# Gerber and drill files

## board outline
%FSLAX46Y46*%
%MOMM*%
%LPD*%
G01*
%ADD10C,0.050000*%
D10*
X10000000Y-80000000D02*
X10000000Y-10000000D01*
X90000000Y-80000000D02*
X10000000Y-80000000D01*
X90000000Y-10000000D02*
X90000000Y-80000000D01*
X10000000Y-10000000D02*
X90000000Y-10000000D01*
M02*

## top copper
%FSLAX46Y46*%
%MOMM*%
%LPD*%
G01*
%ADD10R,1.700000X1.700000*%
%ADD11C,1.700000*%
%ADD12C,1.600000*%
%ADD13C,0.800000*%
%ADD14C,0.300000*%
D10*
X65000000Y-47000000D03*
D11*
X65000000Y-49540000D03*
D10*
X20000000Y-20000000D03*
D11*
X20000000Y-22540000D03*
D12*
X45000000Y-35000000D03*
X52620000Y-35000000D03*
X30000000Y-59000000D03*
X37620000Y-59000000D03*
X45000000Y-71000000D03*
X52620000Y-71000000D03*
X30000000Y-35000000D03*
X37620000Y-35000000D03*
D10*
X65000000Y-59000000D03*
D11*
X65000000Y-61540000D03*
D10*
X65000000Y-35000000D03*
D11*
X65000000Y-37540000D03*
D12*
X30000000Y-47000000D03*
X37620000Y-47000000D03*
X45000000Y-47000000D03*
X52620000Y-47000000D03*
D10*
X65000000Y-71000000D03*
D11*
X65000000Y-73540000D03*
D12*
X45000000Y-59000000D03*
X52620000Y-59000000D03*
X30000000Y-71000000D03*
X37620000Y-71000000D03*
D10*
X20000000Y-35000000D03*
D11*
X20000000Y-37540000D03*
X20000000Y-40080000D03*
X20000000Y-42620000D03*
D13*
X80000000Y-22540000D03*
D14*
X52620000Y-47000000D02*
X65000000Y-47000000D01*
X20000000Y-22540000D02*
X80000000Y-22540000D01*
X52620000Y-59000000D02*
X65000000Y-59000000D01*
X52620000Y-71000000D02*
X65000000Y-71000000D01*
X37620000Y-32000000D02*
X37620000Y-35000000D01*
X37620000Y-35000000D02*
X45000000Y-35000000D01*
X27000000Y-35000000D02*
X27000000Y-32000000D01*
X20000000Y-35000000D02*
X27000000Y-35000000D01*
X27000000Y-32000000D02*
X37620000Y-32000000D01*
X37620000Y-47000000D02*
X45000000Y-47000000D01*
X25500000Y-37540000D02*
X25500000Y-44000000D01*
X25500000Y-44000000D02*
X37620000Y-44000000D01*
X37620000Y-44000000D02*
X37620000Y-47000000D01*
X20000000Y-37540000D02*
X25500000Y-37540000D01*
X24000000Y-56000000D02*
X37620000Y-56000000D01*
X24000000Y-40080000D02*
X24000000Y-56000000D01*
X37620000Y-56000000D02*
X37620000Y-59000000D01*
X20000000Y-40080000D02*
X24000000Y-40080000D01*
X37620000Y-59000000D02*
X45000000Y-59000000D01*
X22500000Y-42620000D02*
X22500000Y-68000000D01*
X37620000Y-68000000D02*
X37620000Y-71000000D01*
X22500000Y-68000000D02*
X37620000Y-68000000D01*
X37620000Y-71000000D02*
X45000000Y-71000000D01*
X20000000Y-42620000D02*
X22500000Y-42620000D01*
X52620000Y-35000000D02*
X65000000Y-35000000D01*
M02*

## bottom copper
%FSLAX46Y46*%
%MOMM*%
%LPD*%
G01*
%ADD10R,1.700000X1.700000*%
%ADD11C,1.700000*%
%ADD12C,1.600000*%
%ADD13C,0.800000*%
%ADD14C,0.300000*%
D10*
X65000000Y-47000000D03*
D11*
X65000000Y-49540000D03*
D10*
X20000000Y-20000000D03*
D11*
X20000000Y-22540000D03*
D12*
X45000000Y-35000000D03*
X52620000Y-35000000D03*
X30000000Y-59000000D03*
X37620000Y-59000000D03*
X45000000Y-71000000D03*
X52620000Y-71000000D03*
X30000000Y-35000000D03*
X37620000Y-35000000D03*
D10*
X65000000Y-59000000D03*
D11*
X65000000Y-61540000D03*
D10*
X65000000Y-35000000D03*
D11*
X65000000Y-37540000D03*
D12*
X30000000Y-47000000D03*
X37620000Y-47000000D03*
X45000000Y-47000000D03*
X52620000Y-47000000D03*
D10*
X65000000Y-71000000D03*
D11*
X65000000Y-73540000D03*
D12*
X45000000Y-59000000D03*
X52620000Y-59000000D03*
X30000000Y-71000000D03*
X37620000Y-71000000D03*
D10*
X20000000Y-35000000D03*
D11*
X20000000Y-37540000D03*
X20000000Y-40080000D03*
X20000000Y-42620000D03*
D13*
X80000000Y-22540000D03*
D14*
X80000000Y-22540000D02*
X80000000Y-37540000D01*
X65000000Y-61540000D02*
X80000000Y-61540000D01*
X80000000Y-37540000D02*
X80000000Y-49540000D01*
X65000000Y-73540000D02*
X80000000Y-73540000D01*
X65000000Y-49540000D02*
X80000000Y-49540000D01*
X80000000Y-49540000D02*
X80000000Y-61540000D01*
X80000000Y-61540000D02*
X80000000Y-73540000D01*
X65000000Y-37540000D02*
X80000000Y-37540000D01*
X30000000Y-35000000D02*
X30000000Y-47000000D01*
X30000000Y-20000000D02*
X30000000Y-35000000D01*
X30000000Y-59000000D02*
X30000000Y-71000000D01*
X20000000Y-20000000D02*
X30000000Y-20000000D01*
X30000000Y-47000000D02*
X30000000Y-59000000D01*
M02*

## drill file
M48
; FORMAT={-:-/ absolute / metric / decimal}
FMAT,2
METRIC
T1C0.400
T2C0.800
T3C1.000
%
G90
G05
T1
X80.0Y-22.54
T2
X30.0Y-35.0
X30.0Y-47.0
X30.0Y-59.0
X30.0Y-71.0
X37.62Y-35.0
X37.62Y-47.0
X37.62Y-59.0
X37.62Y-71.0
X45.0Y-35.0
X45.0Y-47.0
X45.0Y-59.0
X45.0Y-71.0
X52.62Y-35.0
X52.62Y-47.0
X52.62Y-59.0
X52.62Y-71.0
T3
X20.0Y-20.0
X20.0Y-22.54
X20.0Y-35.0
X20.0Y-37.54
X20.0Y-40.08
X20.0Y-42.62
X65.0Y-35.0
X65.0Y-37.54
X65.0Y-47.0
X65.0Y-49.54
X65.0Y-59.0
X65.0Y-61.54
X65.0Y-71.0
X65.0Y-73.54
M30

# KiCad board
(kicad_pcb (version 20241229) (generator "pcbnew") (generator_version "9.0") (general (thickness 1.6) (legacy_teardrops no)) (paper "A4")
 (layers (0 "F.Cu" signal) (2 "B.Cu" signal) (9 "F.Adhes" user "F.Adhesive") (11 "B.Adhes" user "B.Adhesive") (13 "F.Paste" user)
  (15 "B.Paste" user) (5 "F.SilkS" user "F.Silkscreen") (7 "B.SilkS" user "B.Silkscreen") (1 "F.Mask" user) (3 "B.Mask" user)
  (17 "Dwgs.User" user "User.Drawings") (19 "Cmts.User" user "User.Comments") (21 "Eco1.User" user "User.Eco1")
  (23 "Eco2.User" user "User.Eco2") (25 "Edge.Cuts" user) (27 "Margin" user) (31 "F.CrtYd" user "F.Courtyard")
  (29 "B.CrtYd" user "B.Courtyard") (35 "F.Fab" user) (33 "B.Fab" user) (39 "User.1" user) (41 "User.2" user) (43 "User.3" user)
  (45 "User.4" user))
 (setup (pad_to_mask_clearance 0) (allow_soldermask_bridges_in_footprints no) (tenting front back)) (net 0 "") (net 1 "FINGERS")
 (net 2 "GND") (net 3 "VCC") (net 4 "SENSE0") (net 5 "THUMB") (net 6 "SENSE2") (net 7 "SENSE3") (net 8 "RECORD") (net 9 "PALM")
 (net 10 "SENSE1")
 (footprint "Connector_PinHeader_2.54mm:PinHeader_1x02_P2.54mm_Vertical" (layer "F.Cu") (at 65 47)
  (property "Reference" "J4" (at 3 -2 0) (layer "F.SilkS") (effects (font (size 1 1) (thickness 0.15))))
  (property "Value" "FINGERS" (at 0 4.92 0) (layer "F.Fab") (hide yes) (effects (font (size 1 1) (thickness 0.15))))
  (pad "1" thru_hole rect (at 0 0) (size 1.7 1.7) (drill 1) (layers "*.Cu" "*.Mask") (remove_unused_layers no) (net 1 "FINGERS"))
  (pad "2" thru_hole circle (at 0 2.54) (size 1.7 1.7) (drill 1) (layers "*.Cu" "*.Mask") (remove_unused_layers no) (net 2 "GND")))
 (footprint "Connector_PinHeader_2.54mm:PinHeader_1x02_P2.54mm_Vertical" (layer "F.Cu") (at 20 20)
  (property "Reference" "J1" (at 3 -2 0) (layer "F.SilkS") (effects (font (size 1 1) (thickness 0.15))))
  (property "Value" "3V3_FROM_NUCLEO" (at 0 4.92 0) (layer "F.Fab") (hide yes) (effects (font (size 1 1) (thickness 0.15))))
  (pad "1" thru_hole rect (at 0 0) (size 1.7 1.7) (drill 1) (layers "*.Cu" "*.Mask") (remove_unused_layers no) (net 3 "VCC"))
  (pad "2" thru_hole circle (at 0 2.54) (size 1.7 1.7) (drill 1) (layers "*.Cu" "*.Mask") (remove_unused_layers no) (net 2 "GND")))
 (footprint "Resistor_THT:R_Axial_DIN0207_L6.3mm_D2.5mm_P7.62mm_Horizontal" (layer "F.Cu") (at 45 35)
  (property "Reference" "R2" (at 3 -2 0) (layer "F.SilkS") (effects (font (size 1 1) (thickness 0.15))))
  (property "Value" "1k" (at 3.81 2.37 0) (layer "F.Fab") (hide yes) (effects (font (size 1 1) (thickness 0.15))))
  (pad "1" thru_hole circle (at 0 0) (size 1.6 1.6) (drill 0.8) (layers "*.Cu" "*.Mask") (remove_unused_layers no) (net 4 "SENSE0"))
  (pad "2" thru_hole circle (at 7.62 0) (size 1.6 1.6) (drill 0.8) (layers "*.Cu" "*.Mask") (remove_unused_layers no) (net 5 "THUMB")))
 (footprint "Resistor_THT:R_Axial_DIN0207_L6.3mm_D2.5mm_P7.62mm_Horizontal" (layer "F.Cu") (at 30 59)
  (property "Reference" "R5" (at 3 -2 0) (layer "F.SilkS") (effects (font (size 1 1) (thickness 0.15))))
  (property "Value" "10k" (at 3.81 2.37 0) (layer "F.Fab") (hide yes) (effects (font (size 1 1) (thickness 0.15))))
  (pad "1" thru_hole circle (at 0 0) (size 1.6 1.6) (drill 0.8) (layers "*.Cu" "*.Mask") (remove_unused_layers no) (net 3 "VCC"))
  (pad "2" thru_hole circle (at 7.62 0) (size 1.6 1.6) (drill 0.8) (layers "*.Cu" "*.Mask") (remove_unused_layers no) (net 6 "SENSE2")))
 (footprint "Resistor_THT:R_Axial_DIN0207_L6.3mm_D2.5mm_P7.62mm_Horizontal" (layer "F.Cu") (at 45 71)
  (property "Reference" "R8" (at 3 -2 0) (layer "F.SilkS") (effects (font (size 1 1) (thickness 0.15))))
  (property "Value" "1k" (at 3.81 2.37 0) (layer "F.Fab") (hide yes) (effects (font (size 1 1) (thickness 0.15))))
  (pad "1" thru_hole circle (at 0 0) (size 1.6 1.6) (drill 0.8) (layers "*.Cu" "*.Mask") (remove_unused_layers no) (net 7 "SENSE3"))
  (pad "2" thru_hole circle (at 7.62 0) (size 1.6 1.6) (drill 0.8) (layers "*.Cu" "*.Mask") (remove_unused_layers no) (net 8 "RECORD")))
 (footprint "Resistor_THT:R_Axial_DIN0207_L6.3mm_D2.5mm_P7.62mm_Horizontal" (layer "F.Cu") (at 30 35)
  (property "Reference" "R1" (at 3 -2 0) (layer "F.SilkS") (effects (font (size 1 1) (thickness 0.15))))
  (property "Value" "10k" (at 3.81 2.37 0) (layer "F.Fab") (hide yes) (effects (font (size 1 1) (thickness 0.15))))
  (pad "1" thru_hole circle (at 0 0) (size 1.6 1.6) (drill 0.8) (layers "*.Cu" "*.Mask") (remove_unused_layers no) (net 3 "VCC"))
  (pad "2" thru_hole circle (at 7.62 0) (size 1.6 1.6) (drill 0.8) (layers "*.Cu" "*.Mask") (remove_unused_layers no) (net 4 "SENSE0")))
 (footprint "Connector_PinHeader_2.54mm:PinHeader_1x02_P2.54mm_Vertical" (layer "F.Cu") (at 65 59)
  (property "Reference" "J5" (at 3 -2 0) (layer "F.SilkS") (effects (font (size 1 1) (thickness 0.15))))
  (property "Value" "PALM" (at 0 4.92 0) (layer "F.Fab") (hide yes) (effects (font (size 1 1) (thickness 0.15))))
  (pad "1" thru_hole rect (at 0 0) (size 1.7 1.7) (drill 1) (layers "*.Cu" "*.Mask") (remove_unused_layers no) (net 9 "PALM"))
  (pad "2" thru_hole circle (at 0 2.54) (size 1.7 1.7) (drill 1) (layers "*.Cu" "*.Mask") (remove_unused_layers no) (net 2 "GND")))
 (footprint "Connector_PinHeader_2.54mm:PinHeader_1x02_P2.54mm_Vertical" (layer "F.Cu") (at 65 35)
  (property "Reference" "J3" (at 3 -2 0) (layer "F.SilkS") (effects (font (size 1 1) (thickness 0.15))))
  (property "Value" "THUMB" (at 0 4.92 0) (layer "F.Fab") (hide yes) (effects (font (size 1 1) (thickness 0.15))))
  (pad "1" thru_hole rect (at 0 0) (size 1.7 1.7) (drill 1) (layers "*.Cu" "*.Mask") (remove_unused_layers no) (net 5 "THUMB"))
  (pad "2" thru_hole circle (at 0 2.54) (size 1.7 1.7) (drill 1) (layers "*.Cu" "*.Mask") (remove_unused_layers no) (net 2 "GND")))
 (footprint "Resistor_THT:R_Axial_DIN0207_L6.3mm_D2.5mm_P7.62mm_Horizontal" (layer "F.Cu") (at 30 47)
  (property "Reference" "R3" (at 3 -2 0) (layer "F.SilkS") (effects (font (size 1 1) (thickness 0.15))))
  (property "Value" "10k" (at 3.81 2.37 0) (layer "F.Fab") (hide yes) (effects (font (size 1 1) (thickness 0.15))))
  (pad "1" thru_hole circle (at 0 0) (size 1.6 1.6) (drill 0.8) (layers "*.Cu" "*.Mask") (remove_unused_layers no) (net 3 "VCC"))
  (pad "2" thru_hole circle (at 7.62 0) (size 1.6 1.6) (drill 0.8) (layers "*.Cu" "*.Mask") (remove_unused_layers no) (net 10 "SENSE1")))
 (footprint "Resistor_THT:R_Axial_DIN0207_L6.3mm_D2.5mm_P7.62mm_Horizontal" (layer "F.Cu") (at 45 47)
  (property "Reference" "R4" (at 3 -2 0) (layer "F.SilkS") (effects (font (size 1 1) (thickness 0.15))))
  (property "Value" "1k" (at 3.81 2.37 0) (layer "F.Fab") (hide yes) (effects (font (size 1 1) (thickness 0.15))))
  (pad "1" thru_hole circle (at 0 0) (size 1.6 1.6) (drill 0.8) (layers "*.Cu" "*.Mask") (remove_unused_layers no) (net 10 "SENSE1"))
  (pad "2" thru_hole circle (at 7.62 0) (size 1.6 1.6) (drill 0.8) (layers "*.Cu" "*.Mask") (remove_unused_layers no) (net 1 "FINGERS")))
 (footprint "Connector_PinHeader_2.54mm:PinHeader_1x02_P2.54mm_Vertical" (layer "F.Cu") (at 65 71)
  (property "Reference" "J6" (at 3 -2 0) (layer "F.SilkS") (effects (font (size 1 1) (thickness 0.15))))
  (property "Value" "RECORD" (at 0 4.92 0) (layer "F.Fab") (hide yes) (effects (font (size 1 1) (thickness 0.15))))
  (pad "1" thru_hole rect (at 0 0) (size 1.7 1.7) (drill 1) (layers "*.Cu" "*.Mask") (remove_unused_layers no) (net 8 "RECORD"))
  (pad "2" thru_hole circle (at 0 2.54) (size 1.7 1.7) (drill 1) (layers "*.Cu" "*.Mask") (remove_unused_layers no) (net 2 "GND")))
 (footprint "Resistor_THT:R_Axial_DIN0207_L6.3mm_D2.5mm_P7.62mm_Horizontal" (layer "F.Cu") (at 45 59)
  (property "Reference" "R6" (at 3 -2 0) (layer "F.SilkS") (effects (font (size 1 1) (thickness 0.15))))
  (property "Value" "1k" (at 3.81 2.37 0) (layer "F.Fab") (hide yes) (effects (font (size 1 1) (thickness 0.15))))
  (pad "1" thru_hole circle (at 0 0) (size 1.6 1.6) (drill 0.8) (layers "*.Cu" "*.Mask") (remove_unused_layers no) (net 6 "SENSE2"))
  (pad "2" thru_hole circle (at 7.62 0) (size 1.6 1.6) (drill 0.8) (layers "*.Cu" "*.Mask") (remove_unused_layers no) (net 9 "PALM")))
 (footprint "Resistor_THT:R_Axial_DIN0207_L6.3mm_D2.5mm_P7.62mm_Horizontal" (layer "F.Cu") (at 30 71)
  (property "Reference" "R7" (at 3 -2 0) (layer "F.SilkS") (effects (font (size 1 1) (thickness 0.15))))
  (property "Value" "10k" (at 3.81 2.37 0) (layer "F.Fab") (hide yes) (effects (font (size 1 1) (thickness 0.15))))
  (pad "1" thru_hole circle (at 0 0) (size 1.6 1.6) (drill 0.8) (layers "*.Cu" "*.Mask") (remove_unused_layers no) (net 3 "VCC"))
  (pad "2" thru_hole circle (at 7.62 0) (size 1.6 1.6) (drill 0.8) (layers "*.Cu" "*.Mask") (remove_unused_layers no) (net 7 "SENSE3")))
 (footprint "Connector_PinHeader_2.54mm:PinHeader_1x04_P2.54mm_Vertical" (layer "F.Cu") (at 20 35)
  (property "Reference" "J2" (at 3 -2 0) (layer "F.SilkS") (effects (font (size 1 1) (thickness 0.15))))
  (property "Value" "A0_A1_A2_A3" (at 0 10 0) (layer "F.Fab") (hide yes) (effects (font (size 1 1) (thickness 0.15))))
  (pad "1" thru_hole rect (at 0 0) (size 1.7 1.7) (drill 1) (layers "*.Cu" "*.Mask") (remove_unused_layers no) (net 4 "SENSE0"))
  (pad "2" thru_hole circle (at 0 2.54) (size 1.7 1.7) (drill 1) (layers "*.Cu" "*.Mask") (remove_unused_layers no) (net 10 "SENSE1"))
  (pad "3" thru_hole circle (at 0 5.08) (size 1.7 1.7) (drill 1) (layers "*.Cu" "*.Mask") (remove_unused_layers no) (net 6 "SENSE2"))
  (pad "4" thru_hole circle (at 0 7.62) (size 1.7 1.7) (drill 1) (layers "*.Cu" "*.Mask") (remove_unused_layers no) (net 7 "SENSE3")))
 (gr_line (start 10 80) (end 10 10) (stroke (width 0.05) (type default)) (layer "Edge.Cuts"))
 (gr_line (start 90 80) (end 10 80) (stroke (width 0.05) (type default)) (layer "Edge.Cuts"))
 (gr_line (start 90 10) (end 90 80) (stroke (width 0.05) (type default)) (layer "Edge.Cuts"))
 (gr_line (start 10 10) (end 90 10) (stroke (width 0.05) (type default)) (layer "Edge.Cuts"))
 (segment (start 52.62 47) (end 65 47) (width 0.3) (layer "F.Cu") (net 1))
 (segment (start 20 22.54) (end 80 22.54) (width 0.3) (layer "F.Cu") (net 2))
 (via (at 80 22.54) (size 0.8) (drill 0.4) (layers "F.Cu" "B.Cu") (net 2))
 (segment (start 80 22.54) (end 80 37.54) (width 0.3) (layer "B.Cu") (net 2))
 (segment (start 65 61.54) (end 80 61.54) (width 0.3) (layer "B.Cu") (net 2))
 (segment (start 80 37.54) (end 80 49.54) (width 0.3) (layer "B.Cu") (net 2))
 (segment (start 65 73.54) (end 80 73.54) (width 0.3) (layer "B.Cu") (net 2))
 (segment (start 65 49.54) (end 80 49.54) (width 0.3) (layer "B.Cu") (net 2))
 (segment (start 80 49.54) (end 80 61.54) (width 0.3) (layer "B.Cu") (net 2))
 (segment (start 80 61.54) (end 80 73.54) (width 0.3) (layer "B.Cu") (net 2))
 (segment (start 65 37.54) (end 80 37.54) (width 0.3) (layer "B.Cu") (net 2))
 (segment (start 52.62 59) (end 65 59) (width 0.3) (layer "F.Cu") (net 9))
 (segment (start 52.62 71) (end 65 71) (width 0.3) (layer "F.Cu") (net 8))
 (segment (start 37.62 32) (end 37.62 35) (width 0.3) (layer "F.Cu") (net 4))
 (segment (start 37.62 35) (end 45 35) (width 0.3) (layer "F.Cu") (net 4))
 (segment (start 27 35) (end 27 32) (width 0.3) (layer "F.Cu") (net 4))
 (segment (start 20 35) (end 27 35) (width 0.3) (layer "F.Cu") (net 4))
 (segment (start 27 32) (end 37.62 32) (width 0.3) (layer "F.Cu") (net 4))
 (segment (start 37.62 47) (end 45 47) (width 0.3) (layer "F.Cu") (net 10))
 (segment (start 25.5 37.54) (end 25.5 44) (width 0.3) (layer "F.Cu") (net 10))
 (segment (start 25.5 44) (end 37.62 44) (width 0.3) (layer "F.Cu") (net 10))
 (segment (start 37.62 44) (end 37.62 47) (width 0.3) (layer "F.Cu") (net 10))
 (segment (start 20 37.54) (end 25.5 37.54) (width 0.3) (layer "F.Cu") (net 10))
 (segment (start 24 56) (end 37.62 56) (width 0.3) (layer "F.Cu") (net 6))
 (segment (start 24 40.08) (end 24 56) (width 0.3) (layer "F.Cu") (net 6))
 (segment (start 37.62 56) (end 37.62 59) (width 0.3) (layer "F.Cu") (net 6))
 (segment (start 20 40.08) (end 24 40.08) (width 0.3) (layer "F.Cu") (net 6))
 (segment (start 37.62 59) (end 45 59) (width 0.3) (layer "F.Cu") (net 6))
 (segment (start 22.5 42.62) (end 22.5 68) (width 0.3) (layer "F.Cu") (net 7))
 (segment (start 37.62 68) (end 37.62 71) (width 0.3) (layer "F.Cu") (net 7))
 (segment (start 22.5 68) (end 37.62 68) (width 0.3) (layer "F.Cu") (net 7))
 (segment (start 37.62 71) (end 45 71) (width 0.3) (layer "F.Cu") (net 7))
 (segment (start 20 42.62) (end 22.5 42.62) (width 0.3) (layer "F.Cu") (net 7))
 (segment (start 52.62 35) (end 65 35) (width 0.3) (layer "F.Cu") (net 5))
 (segment (start 30 35) (end 30 47) (width 0.3) (layer "B.Cu") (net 3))
 (segment (start 30 20) (end 30 35) (width 0.3) (layer "B.Cu") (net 3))
 (segment (start 30 59) (end 30 71) (width 0.3) (layer "B.Cu") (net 3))
 (segment (start 20 20) (end 30 20) (width 0.3) (layer "B.Cu") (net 3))
 (segment (start 30 47) (end 30 59) (width 0.3) (layer "B.Cu") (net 3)))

